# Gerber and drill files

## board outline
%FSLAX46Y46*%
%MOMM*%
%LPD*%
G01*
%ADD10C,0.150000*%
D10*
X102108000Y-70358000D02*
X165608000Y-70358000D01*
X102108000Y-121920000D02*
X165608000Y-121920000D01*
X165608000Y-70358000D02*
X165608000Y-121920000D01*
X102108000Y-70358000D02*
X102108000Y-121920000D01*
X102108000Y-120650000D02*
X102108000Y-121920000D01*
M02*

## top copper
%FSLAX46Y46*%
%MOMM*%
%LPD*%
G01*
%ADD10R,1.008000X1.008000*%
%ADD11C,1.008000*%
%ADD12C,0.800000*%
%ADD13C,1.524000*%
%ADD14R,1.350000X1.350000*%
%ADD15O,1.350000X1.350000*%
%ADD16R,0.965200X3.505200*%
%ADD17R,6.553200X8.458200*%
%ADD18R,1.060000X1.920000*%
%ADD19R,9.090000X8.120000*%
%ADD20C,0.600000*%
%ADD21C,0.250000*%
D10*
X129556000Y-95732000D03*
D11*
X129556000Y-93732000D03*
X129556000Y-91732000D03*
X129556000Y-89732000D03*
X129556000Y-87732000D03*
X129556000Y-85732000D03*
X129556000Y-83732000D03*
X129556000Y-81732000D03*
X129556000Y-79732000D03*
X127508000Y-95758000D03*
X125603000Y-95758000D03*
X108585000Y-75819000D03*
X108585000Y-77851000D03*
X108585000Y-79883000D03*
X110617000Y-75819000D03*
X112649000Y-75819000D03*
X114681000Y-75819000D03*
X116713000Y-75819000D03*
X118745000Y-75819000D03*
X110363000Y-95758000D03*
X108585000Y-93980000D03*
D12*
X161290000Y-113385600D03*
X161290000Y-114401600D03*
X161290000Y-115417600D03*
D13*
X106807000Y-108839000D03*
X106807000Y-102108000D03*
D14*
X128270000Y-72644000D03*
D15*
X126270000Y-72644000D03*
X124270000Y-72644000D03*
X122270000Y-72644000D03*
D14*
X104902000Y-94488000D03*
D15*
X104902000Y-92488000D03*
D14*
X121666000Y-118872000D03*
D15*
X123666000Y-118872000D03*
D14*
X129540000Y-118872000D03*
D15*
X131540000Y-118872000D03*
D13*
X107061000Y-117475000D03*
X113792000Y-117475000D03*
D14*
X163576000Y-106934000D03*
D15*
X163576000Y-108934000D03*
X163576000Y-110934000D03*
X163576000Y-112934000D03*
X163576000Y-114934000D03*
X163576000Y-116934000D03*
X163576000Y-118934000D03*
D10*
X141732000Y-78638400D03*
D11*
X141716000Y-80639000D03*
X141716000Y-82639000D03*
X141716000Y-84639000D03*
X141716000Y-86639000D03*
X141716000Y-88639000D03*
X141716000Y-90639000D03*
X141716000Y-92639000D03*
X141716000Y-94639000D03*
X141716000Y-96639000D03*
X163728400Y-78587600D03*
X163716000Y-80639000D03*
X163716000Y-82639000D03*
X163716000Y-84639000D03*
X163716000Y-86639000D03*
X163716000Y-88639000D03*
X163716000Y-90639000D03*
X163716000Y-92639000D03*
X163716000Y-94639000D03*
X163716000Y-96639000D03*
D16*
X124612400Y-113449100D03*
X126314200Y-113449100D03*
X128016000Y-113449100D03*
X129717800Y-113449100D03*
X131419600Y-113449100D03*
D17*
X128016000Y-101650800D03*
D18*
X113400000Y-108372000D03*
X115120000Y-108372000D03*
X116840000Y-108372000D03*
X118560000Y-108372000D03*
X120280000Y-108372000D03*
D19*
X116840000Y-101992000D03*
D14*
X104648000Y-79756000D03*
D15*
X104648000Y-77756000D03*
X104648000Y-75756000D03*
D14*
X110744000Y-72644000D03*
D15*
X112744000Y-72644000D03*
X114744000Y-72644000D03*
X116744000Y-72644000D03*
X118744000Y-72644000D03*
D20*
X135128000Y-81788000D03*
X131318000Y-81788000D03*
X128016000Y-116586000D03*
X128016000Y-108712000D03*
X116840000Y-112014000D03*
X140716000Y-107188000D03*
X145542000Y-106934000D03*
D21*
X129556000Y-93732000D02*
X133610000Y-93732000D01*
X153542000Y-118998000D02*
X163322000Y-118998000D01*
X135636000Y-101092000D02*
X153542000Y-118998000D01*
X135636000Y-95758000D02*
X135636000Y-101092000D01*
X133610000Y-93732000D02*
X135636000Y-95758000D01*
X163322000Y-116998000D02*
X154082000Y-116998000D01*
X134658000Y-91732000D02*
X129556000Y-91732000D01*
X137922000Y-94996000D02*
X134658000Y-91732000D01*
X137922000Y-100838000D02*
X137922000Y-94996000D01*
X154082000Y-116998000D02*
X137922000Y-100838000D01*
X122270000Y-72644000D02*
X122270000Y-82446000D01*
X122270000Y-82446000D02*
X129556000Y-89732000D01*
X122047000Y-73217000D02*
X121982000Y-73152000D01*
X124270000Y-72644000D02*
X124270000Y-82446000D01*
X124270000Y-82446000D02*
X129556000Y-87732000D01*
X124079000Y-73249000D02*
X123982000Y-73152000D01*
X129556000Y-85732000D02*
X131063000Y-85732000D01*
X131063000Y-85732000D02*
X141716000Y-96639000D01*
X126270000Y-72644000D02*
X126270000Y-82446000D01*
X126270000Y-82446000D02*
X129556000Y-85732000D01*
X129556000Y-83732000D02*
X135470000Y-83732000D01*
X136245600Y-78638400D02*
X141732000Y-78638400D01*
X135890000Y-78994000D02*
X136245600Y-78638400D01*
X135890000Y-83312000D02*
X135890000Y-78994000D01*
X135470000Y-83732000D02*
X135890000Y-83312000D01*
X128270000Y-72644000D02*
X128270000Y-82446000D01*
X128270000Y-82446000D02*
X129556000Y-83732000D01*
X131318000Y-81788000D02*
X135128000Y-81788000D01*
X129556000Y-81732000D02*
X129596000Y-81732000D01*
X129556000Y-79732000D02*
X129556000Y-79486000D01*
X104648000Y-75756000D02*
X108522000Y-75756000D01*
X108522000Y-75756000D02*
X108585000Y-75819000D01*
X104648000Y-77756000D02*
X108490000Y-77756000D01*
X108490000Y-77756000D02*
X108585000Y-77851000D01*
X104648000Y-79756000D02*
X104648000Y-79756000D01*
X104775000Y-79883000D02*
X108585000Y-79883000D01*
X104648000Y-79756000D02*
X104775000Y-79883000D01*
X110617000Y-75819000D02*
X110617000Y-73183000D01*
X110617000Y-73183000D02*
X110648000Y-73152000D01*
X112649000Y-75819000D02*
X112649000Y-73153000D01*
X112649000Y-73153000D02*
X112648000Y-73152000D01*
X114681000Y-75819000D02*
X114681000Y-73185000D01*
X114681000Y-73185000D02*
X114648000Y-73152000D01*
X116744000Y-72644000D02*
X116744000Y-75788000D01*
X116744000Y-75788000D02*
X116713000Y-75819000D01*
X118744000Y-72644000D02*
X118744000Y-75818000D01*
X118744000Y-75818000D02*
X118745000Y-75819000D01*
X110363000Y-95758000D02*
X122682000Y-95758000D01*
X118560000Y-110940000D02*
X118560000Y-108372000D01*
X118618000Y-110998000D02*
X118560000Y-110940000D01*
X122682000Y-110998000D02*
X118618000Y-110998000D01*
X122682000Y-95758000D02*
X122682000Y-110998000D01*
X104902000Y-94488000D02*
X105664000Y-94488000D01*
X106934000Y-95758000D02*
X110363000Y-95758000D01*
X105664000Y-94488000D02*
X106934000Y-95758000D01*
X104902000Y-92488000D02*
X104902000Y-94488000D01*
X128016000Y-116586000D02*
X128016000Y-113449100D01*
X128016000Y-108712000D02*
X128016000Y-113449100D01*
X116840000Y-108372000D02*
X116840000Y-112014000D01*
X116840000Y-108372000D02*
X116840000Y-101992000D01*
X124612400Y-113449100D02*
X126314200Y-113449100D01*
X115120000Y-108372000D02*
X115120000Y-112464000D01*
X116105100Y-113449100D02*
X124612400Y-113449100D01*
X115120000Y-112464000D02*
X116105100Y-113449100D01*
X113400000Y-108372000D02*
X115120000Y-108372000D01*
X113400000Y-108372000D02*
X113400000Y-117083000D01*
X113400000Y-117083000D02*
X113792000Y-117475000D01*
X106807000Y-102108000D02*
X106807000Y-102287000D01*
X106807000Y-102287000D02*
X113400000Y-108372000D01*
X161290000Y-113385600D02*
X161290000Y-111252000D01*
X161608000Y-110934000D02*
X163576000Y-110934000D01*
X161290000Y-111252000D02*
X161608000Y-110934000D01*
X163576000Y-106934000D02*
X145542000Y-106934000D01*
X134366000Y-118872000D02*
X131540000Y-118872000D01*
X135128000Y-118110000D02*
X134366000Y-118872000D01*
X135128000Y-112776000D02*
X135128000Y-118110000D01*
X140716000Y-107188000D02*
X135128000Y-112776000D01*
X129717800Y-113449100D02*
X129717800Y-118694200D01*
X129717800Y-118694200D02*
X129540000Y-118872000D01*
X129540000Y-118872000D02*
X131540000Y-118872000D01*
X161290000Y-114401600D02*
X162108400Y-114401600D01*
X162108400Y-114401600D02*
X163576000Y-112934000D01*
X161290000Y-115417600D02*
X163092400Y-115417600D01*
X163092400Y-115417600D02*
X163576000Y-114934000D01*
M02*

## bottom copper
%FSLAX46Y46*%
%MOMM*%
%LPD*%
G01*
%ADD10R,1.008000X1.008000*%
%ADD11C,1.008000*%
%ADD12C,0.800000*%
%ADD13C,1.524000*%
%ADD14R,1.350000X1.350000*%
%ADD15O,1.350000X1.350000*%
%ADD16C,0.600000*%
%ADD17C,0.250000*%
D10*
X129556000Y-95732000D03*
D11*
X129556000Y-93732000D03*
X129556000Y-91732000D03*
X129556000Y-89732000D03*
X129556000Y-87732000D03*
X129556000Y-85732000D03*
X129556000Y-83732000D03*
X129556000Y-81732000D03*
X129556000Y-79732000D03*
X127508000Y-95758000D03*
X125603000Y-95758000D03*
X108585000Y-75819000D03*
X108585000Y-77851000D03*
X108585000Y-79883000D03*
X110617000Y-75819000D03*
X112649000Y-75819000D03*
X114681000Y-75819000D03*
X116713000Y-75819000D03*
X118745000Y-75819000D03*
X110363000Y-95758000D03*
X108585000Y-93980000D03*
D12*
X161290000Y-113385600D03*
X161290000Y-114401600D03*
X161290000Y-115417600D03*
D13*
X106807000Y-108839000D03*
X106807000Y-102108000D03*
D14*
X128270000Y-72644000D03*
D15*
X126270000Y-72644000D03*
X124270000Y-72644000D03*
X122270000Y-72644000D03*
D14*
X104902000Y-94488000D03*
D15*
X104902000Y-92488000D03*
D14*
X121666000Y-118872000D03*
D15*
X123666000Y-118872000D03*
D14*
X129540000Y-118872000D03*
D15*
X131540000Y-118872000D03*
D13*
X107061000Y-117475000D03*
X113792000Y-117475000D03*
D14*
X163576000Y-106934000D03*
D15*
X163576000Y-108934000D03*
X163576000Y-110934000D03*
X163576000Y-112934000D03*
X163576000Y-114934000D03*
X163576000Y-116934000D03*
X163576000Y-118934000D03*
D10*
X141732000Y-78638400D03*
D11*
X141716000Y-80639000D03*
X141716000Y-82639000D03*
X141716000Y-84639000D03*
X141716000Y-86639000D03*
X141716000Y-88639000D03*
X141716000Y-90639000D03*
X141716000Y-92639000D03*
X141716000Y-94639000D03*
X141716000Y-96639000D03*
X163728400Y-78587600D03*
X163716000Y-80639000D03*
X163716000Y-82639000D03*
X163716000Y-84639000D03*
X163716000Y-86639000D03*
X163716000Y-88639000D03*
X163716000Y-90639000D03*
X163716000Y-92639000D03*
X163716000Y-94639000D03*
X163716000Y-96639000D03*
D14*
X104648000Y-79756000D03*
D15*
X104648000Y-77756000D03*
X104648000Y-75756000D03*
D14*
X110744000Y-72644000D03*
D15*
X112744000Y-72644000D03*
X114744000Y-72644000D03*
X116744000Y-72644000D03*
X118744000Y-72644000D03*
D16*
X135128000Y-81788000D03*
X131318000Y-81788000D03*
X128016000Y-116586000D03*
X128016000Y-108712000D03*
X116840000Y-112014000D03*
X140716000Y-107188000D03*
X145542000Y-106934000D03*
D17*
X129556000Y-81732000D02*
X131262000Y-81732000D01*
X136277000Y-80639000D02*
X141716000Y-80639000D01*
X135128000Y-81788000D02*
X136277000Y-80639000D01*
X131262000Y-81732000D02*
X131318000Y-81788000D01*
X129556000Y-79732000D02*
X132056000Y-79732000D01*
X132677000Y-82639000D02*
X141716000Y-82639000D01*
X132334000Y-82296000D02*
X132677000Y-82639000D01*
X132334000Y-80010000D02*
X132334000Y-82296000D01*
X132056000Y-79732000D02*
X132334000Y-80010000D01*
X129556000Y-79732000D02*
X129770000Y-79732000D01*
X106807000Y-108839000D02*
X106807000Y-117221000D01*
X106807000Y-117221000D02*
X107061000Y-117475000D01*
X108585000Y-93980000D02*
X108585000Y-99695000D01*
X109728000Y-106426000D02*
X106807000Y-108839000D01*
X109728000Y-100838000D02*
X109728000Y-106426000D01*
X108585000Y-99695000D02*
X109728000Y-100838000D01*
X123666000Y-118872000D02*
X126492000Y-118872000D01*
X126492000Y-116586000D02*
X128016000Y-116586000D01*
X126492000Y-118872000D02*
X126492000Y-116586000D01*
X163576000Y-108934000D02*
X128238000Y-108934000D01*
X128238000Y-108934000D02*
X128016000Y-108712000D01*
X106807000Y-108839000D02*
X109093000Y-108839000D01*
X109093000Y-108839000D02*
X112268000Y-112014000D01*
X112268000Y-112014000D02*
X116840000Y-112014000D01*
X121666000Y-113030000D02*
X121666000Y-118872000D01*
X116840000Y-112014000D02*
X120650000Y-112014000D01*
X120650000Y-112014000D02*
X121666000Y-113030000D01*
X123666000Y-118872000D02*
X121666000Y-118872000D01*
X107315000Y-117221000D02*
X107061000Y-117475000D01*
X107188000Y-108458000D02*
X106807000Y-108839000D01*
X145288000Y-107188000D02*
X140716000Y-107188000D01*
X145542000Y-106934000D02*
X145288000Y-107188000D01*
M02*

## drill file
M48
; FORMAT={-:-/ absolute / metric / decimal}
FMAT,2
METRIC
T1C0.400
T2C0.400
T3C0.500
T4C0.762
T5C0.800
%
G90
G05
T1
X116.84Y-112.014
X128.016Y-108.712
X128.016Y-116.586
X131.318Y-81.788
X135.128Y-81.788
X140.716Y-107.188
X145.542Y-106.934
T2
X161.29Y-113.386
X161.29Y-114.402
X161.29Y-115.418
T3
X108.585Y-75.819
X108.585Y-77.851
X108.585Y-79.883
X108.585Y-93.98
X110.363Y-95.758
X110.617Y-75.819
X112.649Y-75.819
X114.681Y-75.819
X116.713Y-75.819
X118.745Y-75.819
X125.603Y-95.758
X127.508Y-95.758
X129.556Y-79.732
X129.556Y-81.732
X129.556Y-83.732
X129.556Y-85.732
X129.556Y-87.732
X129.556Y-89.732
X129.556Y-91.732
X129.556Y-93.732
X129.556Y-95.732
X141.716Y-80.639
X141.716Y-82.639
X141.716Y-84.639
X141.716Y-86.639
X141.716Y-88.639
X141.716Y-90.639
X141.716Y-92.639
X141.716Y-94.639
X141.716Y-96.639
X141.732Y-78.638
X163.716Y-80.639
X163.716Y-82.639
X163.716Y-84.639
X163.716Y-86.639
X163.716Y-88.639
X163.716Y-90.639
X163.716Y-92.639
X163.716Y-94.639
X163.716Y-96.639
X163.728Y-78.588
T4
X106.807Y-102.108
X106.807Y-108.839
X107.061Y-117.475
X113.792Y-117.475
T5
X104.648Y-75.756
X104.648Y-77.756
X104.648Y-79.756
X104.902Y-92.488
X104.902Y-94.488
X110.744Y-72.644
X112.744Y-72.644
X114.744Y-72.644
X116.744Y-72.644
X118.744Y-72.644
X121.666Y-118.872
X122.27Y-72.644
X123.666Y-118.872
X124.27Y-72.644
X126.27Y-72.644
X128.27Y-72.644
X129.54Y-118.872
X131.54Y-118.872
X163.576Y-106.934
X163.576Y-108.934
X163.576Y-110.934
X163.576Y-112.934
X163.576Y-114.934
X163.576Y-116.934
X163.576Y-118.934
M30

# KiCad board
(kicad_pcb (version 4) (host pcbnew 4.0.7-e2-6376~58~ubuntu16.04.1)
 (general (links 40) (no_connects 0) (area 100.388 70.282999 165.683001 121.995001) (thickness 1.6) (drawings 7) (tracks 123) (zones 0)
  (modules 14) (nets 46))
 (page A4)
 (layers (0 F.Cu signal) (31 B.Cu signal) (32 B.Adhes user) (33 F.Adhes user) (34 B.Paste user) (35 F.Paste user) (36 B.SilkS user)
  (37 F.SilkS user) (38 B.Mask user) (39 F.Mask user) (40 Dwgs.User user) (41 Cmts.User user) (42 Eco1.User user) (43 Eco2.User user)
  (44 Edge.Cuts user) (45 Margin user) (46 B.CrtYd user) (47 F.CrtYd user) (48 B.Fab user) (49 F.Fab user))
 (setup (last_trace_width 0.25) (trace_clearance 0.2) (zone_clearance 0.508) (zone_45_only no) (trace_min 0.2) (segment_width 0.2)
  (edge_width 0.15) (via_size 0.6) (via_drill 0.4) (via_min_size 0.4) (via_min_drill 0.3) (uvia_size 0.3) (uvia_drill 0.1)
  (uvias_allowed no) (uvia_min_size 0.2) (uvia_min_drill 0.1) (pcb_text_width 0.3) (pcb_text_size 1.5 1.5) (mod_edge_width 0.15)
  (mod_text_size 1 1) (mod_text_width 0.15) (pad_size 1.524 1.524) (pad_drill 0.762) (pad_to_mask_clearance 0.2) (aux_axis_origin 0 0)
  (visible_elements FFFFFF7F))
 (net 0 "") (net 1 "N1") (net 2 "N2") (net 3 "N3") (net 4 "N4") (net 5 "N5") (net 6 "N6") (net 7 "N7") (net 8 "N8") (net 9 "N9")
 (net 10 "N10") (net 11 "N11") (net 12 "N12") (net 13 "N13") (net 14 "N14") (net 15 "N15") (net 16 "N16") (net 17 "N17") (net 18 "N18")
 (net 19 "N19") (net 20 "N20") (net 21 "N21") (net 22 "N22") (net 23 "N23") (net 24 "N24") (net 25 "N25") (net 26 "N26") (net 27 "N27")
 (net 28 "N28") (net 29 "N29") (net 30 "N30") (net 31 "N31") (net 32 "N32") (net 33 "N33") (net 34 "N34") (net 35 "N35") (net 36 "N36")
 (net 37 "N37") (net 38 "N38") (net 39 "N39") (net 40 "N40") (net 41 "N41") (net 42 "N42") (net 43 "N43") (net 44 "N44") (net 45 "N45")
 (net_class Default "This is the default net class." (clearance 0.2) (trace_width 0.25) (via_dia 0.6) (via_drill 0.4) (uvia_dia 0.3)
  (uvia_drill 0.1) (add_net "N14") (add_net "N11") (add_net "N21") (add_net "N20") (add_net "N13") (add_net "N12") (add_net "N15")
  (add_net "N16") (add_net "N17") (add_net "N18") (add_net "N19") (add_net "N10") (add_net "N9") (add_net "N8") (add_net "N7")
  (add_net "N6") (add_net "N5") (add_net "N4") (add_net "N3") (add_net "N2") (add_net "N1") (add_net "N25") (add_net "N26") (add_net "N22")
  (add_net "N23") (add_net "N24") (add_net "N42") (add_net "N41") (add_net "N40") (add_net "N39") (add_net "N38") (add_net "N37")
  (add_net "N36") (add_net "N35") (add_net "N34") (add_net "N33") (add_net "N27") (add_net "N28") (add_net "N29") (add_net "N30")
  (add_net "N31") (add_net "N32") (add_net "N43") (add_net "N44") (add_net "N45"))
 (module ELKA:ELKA (layer F.Cu) (at 118.11 72.39 180)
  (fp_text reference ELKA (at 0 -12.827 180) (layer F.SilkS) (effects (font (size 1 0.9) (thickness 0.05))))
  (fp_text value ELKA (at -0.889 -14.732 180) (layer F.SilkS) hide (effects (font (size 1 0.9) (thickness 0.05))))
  (pad I thru_hole rect (at -11.446 -23.342 180) (size 1.008 1.008) (drill 0.5) (layers *.Cu *.Mask F.SilkS) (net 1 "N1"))
  (pad H thru_hole circle (at -11.446 -21.342 180) (size 1.008 1.008) (drill 0.5) (layers *.Cu *.Mask F.SilkS) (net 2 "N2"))
  (pad G thru_hole circle (at -11.446 -19.342 180) (size 1.008 1.008) (drill 0.5) (layers *.Cu *.Mask F.SilkS) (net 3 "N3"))
  (pad F thru_hole circle (at -11.446 -17.342 180) (size 1.008 1.008) (drill 0.5) (layers *.Cu *.Mask F.SilkS) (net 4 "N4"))
  (pad E thru_hole circle (at -11.446 -15.342 180) (size 1.008 1.008) (drill 0.5) (layers *.Cu *.Mask F.SilkS) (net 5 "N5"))
  (pad D thru_hole circle (at -11.446 -13.342 180) (size 1.008 1.008) (drill 0.5) (layers *.Cu *.Mask F.SilkS) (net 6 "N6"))
  (pad C thru_hole circle (at -11.446 -11.342 180) (size 1.008 1.008) (drill 0.5) (layers *.Cu *.Mask F.SilkS) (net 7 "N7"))
  (pad B thru_hole circle (at -11.446 -9.342 180) (size 1.008 1.008) (drill 0.5) (layers *.Cu *.Mask F.SilkS) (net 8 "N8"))
  (pad A thru_hole circle (at -11.446 -7.342 180) (size 1.008 1.008) (drill 0.5) (layers *.Cu *.Mask F.SilkS) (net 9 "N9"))
  (pad 9 thru_hole circle (at -9.398 -23.368 180) (size 1.008 1.008) (drill 0.5) (layers *.Cu *.Mask F.SilkS) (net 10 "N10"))
  (pad 10 thru_hole circle (at -7.493 -23.368 180) (size 1.008 1.008) (drill 0.5) (layers *.Cu *.Mask F.SilkS) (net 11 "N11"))
  (pad 3 thru_hole circle (at 9.525 -3.429 180) (size 1.008 1.008) (drill 0.5) (layers *.Cu *.Mask F.SilkS) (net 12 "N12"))
  (pad 2 thru_hole circle (at 9.525 -5.461 180) (size 1.008 1.008) (drill 0.5) (layers *.Cu *.Mask F.SilkS) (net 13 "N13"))
  (pad 1 thru_hole circle (at 9.525 -7.493 180) (size 1.008 1.008) (drill 0.5) (layers *.Cu *.Mask F.SilkS) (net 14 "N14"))
  (pad 4 thru_hole circle (at 7.493 -3.429 180) (size 1.008 1.008) (drill 0.5) (layers *.Cu *.Mask F.SilkS) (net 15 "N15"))
  (pad 5 thru_hole circle (at 5.461 -3.429 180) (size 1.008 1.008) (drill 0.5) (layers *.Cu *.Mask F.SilkS) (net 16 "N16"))
  (pad 6 thru_hole circle (at 3.429 -3.429 180) (size 1.008 1.008) (drill 0.5) (layers *.Cu *.Mask F.SilkS) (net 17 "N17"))
  (pad 7 thru_hole circle (at 1.397 -3.429 180) (size 1.008 1.008) (drill 0.5) (layers *.Cu *.Mask F.SilkS) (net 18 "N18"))
  (pad 8 thru_hole circle (at -0.635 -3.429 180) (size 1.008 1.008) (drill 0.5) (layers *.Cu *.Mask F.SilkS) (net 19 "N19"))
  (pad 12 thru_hole circle (at 7.747 -23.368 180) (size 1.008 1.008) (drill 0.5) (layers *.Cu *.Mask F.SilkS) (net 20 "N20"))
  (pad 11 thru_hole circle (at 9.525 -21.59 180) (size 1.008 1.008) (drill 0.5) (layers *.Cu *.Mask F.SilkS) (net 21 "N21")))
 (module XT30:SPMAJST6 (layer F.Cu) (at 164.084 115.316 270)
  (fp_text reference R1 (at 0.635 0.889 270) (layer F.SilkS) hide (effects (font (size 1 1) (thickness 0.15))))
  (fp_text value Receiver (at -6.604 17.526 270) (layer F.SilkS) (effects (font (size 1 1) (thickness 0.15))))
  (pad 1 thru_hole circle (at -1.9304 2.794 270) (size 0.8 0.8) (drill 0.4) (layers *.Cu *.Mask) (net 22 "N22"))
  (pad 2 thru_hole circle (at -0.9144 2.794 270) (size 0.8 0.8) (drill 0.4) (layers *.Cu *.Mask) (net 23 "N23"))
  (pad 3 thru_hole circle (at 0.1016 2.794 270) (size 0.8 0.8) (drill 0.4) (layers *.Cu *.Mask) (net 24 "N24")))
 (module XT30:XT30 (layer F.Cu) (at 100.838 107.442 90)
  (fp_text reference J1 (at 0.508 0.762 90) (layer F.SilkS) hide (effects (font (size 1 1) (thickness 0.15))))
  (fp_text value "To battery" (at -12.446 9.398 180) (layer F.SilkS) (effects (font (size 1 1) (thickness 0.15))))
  (pad 1 thru_hole circle (at -1.397 5.969 90) (size 1.524 1.524) (drill 0.762) (layers *.Cu *.Mask) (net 21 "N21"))
  (pad 2 thru_hole circle (at 5.334 5.969 90) (size 1.524 1.524) (drill 0.762) (layers *.Cu *.Mask) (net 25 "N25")))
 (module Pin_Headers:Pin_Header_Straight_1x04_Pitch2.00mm (layer F.Cu) (at 128.27 72.644 270)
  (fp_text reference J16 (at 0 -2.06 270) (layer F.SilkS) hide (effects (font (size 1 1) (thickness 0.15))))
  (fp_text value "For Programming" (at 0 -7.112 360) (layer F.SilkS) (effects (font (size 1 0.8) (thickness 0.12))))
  (pad 1 thru_hole rect (at 0 0 270) (size 1.35 1.35) (drill 0.8) (layers *.Cu *.Mask) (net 7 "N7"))
  (pad 2 thru_hole oval (at 0 2 270) (size 1.35 1.35) (drill 0.8) (layers *.Cu *.Mask) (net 6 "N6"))
  (pad 3 thru_hole oval (at 0 4 270) (size 1.35 1.35) (drill 0.8) (layers *.Cu *.Mask) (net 5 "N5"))
  (pad 4 thru_hole oval (at 0 6 270) (size 1.35 1.35) (drill 0.8) (layers *.Cu *.Mask) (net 4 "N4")))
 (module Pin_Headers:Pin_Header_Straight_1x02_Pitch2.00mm (layer F.Cu) (at 104.902 94.488 180)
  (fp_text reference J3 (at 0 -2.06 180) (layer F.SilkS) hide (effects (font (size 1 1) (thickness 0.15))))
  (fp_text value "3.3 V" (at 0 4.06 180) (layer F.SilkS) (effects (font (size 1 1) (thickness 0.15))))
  (pad 1 thru_hole rect (at 0 0 180) (size 1.35 1.35) (drill 0.8) (layers *.Cu *.Mask) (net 20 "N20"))
  (pad 2 thru_hole oval (at 0 2 180) (size 1.35 1.35) (drill 0.8) (layers *.Cu *.Mask) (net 20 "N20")))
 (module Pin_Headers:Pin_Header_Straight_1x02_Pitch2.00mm (layer F.Cu) (at 121.666 118.872 90)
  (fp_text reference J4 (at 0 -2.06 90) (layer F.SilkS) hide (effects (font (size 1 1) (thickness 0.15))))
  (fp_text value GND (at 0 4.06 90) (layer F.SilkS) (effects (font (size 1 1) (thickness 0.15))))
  (pad 1 thru_hole rect (at 0 0 90) (size 1.35 1.35) (drill 0.8) (layers *.Cu *.Mask) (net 21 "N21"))
  (pad 2 thru_hole oval (at 0 2 90) (size 1.35 1.35) (drill 0.8) (layers *.Cu *.Mask) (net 21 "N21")))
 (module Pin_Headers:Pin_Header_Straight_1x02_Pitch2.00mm (layer F.Cu) (at 129.54 118.872 90)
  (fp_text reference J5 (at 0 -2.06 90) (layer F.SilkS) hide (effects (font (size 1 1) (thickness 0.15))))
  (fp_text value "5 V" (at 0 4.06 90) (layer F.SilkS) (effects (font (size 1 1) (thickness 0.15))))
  (pad 1 thru_hole rect (at 0 0 90) (size 1.35 1.35) (drill 0.8) (layers *.Cu *.Mask) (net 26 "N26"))
  (pad 2 thru_hole oval (at 0 2 90) (size 1.35 1.35) (drill 0.8) (layers *.Cu *.Mask) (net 26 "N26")))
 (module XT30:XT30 (layer F.Cu) (at 108.458 111.506)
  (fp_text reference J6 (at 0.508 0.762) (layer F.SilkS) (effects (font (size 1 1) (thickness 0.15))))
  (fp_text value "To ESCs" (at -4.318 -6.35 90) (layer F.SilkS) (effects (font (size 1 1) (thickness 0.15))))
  (pad 1 thru_hole circle (at -1.397 5.969) (size 1.524 1.524) (drill 0.762) (layers *.Cu *.Mask) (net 21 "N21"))
  (pad 2 thru_hole circle (at 5.334 5.969) (size 1.524 1.524) (drill 0.762) (layers *.Cu *.Mask) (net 25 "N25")))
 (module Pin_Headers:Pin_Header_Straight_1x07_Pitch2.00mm (layer F.Cu) (at 163.576 106.934)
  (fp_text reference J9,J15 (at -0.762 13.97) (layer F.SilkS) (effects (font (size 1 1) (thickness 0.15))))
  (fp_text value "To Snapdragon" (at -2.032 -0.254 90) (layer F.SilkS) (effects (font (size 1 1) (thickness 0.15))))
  (pad 1 thru_hole rect (at 0 0) (size 1.35 1.35) (drill 0.8) (layers *.Cu *.Mask) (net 26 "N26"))
  (pad 2 thru_hole oval (at 0 2) (size 1.35 1.35) (drill 0.8) (layers *.Cu *.Mask) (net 21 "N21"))
  (pad 3 thru_hole oval (at 0 4) (size 1.35 1.35) (drill 0.8) (layers *.Cu *.Mask) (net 22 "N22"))
  (pad 4 thru_hole oval (at 0 6) (size 1.35 1.35) (drill 0.8) (layers *.Cu *.Mask) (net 23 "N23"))
  (pad 5 thru_hole oval (at 0 8) (size 1.35 1.35) (drill 0.8) (layers *.Cu *.Mask) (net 24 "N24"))
  (pad 6 thru_hole oval (at 0 10) (size 1.35 1.35) (drill 0.8) (layers *.Cu *.Mask) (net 3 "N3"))
  (pad 7 thru_hole oval (at 0 12) (size 1.35 1.35) (drill 0.8) (layers *.Cu *.Mask) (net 2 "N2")))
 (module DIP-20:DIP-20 (layer F.Cu) (at 140.462 104.648)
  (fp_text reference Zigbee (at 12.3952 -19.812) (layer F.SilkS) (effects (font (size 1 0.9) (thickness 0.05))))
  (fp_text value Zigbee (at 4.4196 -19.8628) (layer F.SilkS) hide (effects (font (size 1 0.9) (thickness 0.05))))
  (pad 1 thru_hole rect (at 1.27 -26.0096) (size 1.008 1.008) (drill 0.5) (layers *.Cu *.Mask F.SilkS) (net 7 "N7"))
  (pad 2 thru_hole circle (at 1.254 -24.009) (size 1.008 1.008) (drill 0.5) (layers *.Cu *.Mask F.SilkS) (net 8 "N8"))
  (pad 3 thru_hole circle (at 1.254 -22.009) (size 1.008 1.008) (drill 0.5) (layers *.Cu *.Mask F.SilkS) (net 9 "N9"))
  (pad 4 thru_hole circle (at 1.254 -20.009) (size 1.008 1.008) (drill 0.5) (layers *.Cu *.Mask F.SilkS) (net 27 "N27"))
  (pad 5 thru_hole circle (at 1.254 -18.009) (size 1.008 1.008) (drill 0.5) (layers *.Cu *.Mask F.SilkS) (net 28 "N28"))
  (pad 6 thru_hole circle (at 1.254 -16.009) (size 1.008 1.008) (drill 0.5) (layers *.Cu *.Mask F.SilkS) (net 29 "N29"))
  (pad 7 thru_hole circle (at 1.254 -14.009) (size 1.008 1.008) (drill 0.5) (layers *.Cu *.Mask F.SilkS) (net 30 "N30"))
  (pad 8 thru_hole circle (at 1.254 -12.009) (size 1.008 1.008) (drill 0.5) (layers *.Cu *.Mask F.SilkS) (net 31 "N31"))
  (pad 9 thru_hole circle (at 1.254 -10.009) (size 1.008 1.008) (drill 0.5) (layers *.Cu *.Mask F.SilkS) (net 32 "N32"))
  (pad 10 thru_hole circle (at 1.254 -8.009) (size 1.008 1.008) (drill 0.5) (layers *.Cu *.Mask F.SilkS) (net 6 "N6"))
  (pad 20 thru_hole circle (at 23.2664 -26.0604) (size 1.008 1.008) (drill 0.5) (layers *.Cu *.Mask F.SilkS) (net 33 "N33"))
  (pad 19 thru_hole circle (at 23.254 -24.009) (size 1.008 1.008) (drill 0.5) (layers *.Cu *.Mask F.SilkS) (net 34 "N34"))
  (pad 18 thru_hole circle (at 23.254 -22.009) (size 1.008 1.008) (drill 0.5) (layers *.Cu *.Mask F.SilkS) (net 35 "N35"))
  (pad 17 thru_hole circle (at 23.254 -20.009) (size 1.008 1.008) (drill 0.5) (layers *.Cu *.Mask F.SilkS) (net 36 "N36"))
  (pad 16 thru_hole circle (at 23.254 -18.009) (size 1.008 1.008) (drill 0.5) (layers *.Cu *.Mask F.SilkS) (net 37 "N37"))
  (pad 15 thru_hole circle (at 23.254 -16.009) (size 1.008 1.008) (drill 0.5) (layers *.Cu *.Mask F.SilkS) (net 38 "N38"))
  (pad 14 thru_hole circle (at 23.254 -14.009) (size 1.008 1.008) (drill 0.5) (layers *.Cu *.Mask F.SilkS) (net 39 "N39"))
  (pad 13 thru_hole circle (at 23.254 -12.009) (size 1.008 1.008) (drill 0.5) (layers *.Cu *.Mask F.SilkS) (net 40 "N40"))
  (pad 12 thru_hole circle (at 23.254 -10.009) (size 1.008 1.008) (drill 0.5) (layers *.Cu *.Mask F.SilkS) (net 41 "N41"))
  (pad 11 thru_hole circle (at 23.254 -8.009) (size 1.008 1.008) (drill 0.5) (layers *.Cu *.Mask F.SilkS) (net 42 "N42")))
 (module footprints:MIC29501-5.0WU (layer F.Cu) (at 128.016 104.394)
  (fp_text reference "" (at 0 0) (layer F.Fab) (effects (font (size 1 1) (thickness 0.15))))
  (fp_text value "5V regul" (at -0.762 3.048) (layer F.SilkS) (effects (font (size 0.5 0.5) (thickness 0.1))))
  (pad 1 smd rect (at -3.4036 9.0551) (size 0.9652 3.5052) (layers F.Cu F.Paste F.Mask) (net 25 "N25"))
  (pad 2 smd rect (at -1.7018 9.0551) (size 0.9652 3.5052) (layers F.Cu F.Paste F.Mask) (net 25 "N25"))
  (pad 3 smd rect (at 0 9.0551) (size 0.9652 3.5052) (layers F.Cu F.Paste F.Mask) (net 21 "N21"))
  (pad 4 smd rect (at 1.7018 9.0551) (size 0.9652 3.5052) (layers F.Cu F.Paste F.Mask) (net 26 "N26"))
  (pad 5 smd rect (at 3.4036 9.0551) (size 0.9652 3.5052) (layers F.Cu F.Paste F.Mask) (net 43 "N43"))
  (pad 6 smd rect (at 0 -2.7432) (size 6.5532 8.4582) (layers F.Cu F.Paste F.Mask) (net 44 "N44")))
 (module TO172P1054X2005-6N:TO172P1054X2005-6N (layer F.Cu) (at 116.84 103.632)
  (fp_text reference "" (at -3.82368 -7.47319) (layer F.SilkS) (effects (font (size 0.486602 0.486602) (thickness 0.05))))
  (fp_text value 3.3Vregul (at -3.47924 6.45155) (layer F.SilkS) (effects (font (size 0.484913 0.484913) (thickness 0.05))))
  (pad 1 smd rect (at -3.44 4.74 90) (size 1.92 1.06) (layers F.Cu F.Paste F.Mask) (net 25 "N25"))
  (pad 2 smd rect (at -1.72 4.74 90) (size 1.92 1.06) (layers F.Cu F.Paste F.Mask) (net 25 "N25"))
  (pad 3 smd rect (at 0 4.74 90) (size 1.92 1.06) (layers F.Cu F.Paste F.Mask) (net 21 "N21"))
  (pad 4 smd rect (at 1.72 4.74 90) (size 1.92 1.06) (layers F.Cu F.Paste F.Mask) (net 20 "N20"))
  (pad 5 smd rect (at 3.44 4.74 90) (size 1.92 1.06) (layers F.Cu F.Paste F.Mask) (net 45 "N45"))
  (pad 6 smd rect (at 0 -1.64 90) (size 8.12 9.09) (layers F.Cu F.Paste F.Mask) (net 21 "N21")))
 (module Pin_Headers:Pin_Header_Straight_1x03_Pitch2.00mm (layer F.Cu) (at 104.648 79.756 180)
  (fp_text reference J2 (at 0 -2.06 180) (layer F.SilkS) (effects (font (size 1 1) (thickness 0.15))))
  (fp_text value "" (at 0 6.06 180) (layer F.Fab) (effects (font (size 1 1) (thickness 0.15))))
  (pad 1 thru_hole rect (at 0 0 180) (size 1.35 1.35) (drill 0.8) (layers *.Cu *.Mask) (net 14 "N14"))
  (pad 2 thru_hole oval (at 0 2 180) (size 1.35 1.35) (drill 0.8) (layers *.Cu *.Mask) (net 13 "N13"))
  (pad 3 thru_hole oval (at 0 4 180) (size 1.35 1.35) (drill 0.8) (layers *.Cu *.Mask) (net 12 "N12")))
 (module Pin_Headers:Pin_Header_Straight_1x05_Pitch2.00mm (layer F.Cu) (at 110.744 72.644 90)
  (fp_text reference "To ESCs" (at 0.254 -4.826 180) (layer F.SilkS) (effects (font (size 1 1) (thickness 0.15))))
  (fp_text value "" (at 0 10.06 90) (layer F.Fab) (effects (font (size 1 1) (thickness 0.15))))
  (pad 1 thru_hole rect (at 0 0 90) (size 1.35 1.35) (drill 0.8) (layers *.Cu *.Mask) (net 15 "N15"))
  (pad 2 thru_hole oval (at 0 2 90) (size 1.35 1.35) (drill 0.8) (layers *.Cu *.Mask) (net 16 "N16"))
  (pad 3 thru_hole oval (at 0 4 90) (size 1.35 1.35) (drill 0.8) (layers *.Cu *.Mask) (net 17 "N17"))
  (pad 4 thru_hole oval (at 0 6 90) (size 1.35 1.35) (drill 0.8) (layers *.Cu *.Mask) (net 18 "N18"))
  (pad 5 thru_hole oval (at 0 8 90) (size 1.35 1.35) (drill 0.8) (layers *.Cu *.Mask) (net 19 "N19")))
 (gr_line (start 102.108 70.358) (end 165.608 70.358) (angle 90) (layer Edge.Cuts) (width 0.15))
 (gr_line (start 102.108 121.92) (end 165.608 121.92) (angle 90) (layer Edge.Cuts) (width 0.15))
 (gr_line (start 165.608 70.358) (end 165.608 121.92) (angle 90) (layer Edge.Cuts) (width 0.15))
 (gr_line (start 102.108 70.358) (end 102.108 121.92) (angle 90) (layer Edge.Cuts) (width 0.15))
 (gr_line (start 102.108 120.65) (end 102.108 121.92) (angle 90) (layer Edge.Cuts) (width 0.15))
 (segment (start 129.556 93.732) (end 133.61 93.732) (width 0.25) (layer F.Cu) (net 2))
 (segment (start 153.542 118.998) (end 163.322 118.998) (width 0.25) (layer F.Cu) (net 2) (status 20))
 (segment (start 135.636 101.092) (end 153.542 118.998) (width 0.25) (layer F.Cu) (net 2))
 (segment (start 135.636 95.758) (end 135.636 101.092) (width 0.25) (layer F.Cu) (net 2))
 (segment (start 133.61 93.732) (end 135.636 95.758) (width 0.25) (layer F.Cu) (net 2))
 (segment (start 163.322 116.998) (end 154.082 116.998) (width 0.25) (layer F.Cu) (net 3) (status 10))
 (segment (start 134.658 91.732) (end 129.556 91.732) (width 0.25) (layer F.Cu) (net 3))
 (segment (start 137.922 94.996) (end 134.658 91.732) (width 0.25) (layer F.Cu) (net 3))
 (segment (start 137.922 100.838) (end 137.922 94.996) (width 0.25) (layer F.Cu) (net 3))
 (segment (start 154.082 116.998) (end 137.922 100.838) (width 0.25) (layer F.Cu) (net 3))
 (segment (start 122.27 72.644) (end 122.27 82.446) (width 0.25) (layer F.Cu) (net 4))
 (segment (start 122.27 82.446) (end 129.556 89.732) (width 0.25) (layer F.Cu) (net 4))
 (segment (start 122.047 73.217) (end 121.982 73.152) (width 0.25) (layer F.Cu) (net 4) (status 30))
 (segment (start 124.27 72.644) (end 124.27 82.446) (width 0.25) (layer F.Cu) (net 5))
 (segment (start 124.27 82.446) (end 129.556 87.732) (width 0.25) (layer F.Cu) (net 5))
 (segment (start 124.079 73.249) (end 123.982 73.152) (width 0.25) (layer F.Cu) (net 5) (status 30))
 (segment (start 129.556 85.732) (end 131.063 85.732) (width 0.25) (layer F.Cu) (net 6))
 (segment (start 131.063 85.732) (end 141.716 96.639) (width 0.25) (layer F.Cu) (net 6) (status 20))
 (segment (start 126.27 72.644) (end 126.27 82.446) (width 0.25) (layer F.Cu) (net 6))
 (segment (start 126.27 82.446) (end 129.556 85.732) (width 0.25) (layer F.Cu) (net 6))
 (segment (start 129.556 83.732) (end 135.47 83.732) (width 0.25) (layer F.Cu) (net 7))
 (segment (start 136.2456 78.6384) (end 141.732 78.6384) (width 0.25) (layer F.Cu) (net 7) (status 20))
 (segment (start 135.89 78.994) (end 136.2456 78.6384) (width 0.25) (layer F.Cu) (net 7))
 (segment (start 135.89 83.312) (end 135.89 78.994) (width 0.25) (layer F.Cu) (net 7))
 (segment (start 135.47 83.732) (end 135.89 83.312) (width 0.25) (layer F.Cu) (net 7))
 (segment (start 128.27 72.644) (end 128.27 82.446) (width 0.25) (layer F.Cu) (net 7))
 (segment (start 128.27 82.446) (end 129.556 83.732) (width 0.25) (layer F.Cu) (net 7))
 (segment (start 129.556 81.732) (end 131.262 81.732) (width 0.25) (layer B.Cu) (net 8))
 (segment (start 136.277 80.639) (end 141.716 80.639) (width 0.25) (layer B.Cu) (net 8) (status 20))
 (segment (start 135.128 81.788) (end 136.277 80.639) (width 0.25) (layer B.Cu) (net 8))
 (via (at 135.128 81.788) (size 0.6) (drill 0.4) (layers F.Cu B.Cu) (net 8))
 (segment (start 131.318 81.788) (end 135.128 81.788) (width 0.25) (layer F.Cu) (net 8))
 (via (at 131.318 81.788) (size 0.6) (drill 0.4) (layers F.Cu B.Cu) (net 8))
 (segment (start 131.262 81.732) (end 131.318 81.788) (width 0.25) (layer B.Cu) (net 8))
 (segment (start 129.556 81.732) (end 129.596 81.732) (width 0.25) (layer F.Cu) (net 8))
 (segment (start 129.556 79.732) (end 132.056 79.732) (width 0.25) (layer B.Cu) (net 9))
 (segment (start 132.677 82.639) (end 141.716 82.639) (width 0.25) (layer B.Cu) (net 9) (status 20))
 (segment (start 132.334 82.296) (end 132.677 82.639) (width 0.25) (layer B.Cu) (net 9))
 (segment (start 132.334 80.01) (end 132.334 82.296) (width 0.25) (layer B.Cu) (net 9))
 (segment (start 132.056 79.732) (end 132.334 80.01) (width 0.25) (layer B.Cu) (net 9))
 (segment (start 129.556 79.732) (end 129.556 79.486) (width 0.25) (layer F.Cu) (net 9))
 (segment (start 129.556 79.732) (end 129.77 79.732) (width 0.25) (layer B.Cu) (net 9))
 (segment (start 104.648 75.756) (end 108.522 75.756) (width 0.25) (layer F.Cu) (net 12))
 (segment (start 108.522 75.756) (end 108.585 75.819) (width 0.25) (layer F.Cu) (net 12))
 (segment (start 104.648 77.756) (end 108.49 77.756) (width 0.25) (layer F.Cu) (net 13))
 (segment (start 108.49 77.756) (end 108.585 77.851) (width 0.25) (layer F.Cu) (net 13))
 (segment (start 104.648 79.756) (end 104.648 79.756) (width 0.25) (layer F.Cu) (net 14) (status 10))
 (segment (start 104.775 79.883) (end 108.585 79.883) (width 0.25) (layer F.Cu) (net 14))
 (segment (start 104.648 79.756) (end 104.775 79.883) (width 0.25) (layer F.Cu) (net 14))
 (segment (start 110.617 75.819) (end 110.617 73.183) (width 0.25) (layer F.Cu) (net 15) (status 20))
 (segment (start 110.617 73.183) (end 110.648 73.152) (width 0.25) (layer F.Cu) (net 15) (status 30))
 (segment (start 112.649 75.819) (end 112.649 73.153) (width 0.25) (layer F.Cu) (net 16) (status 20))
 (segment (start 112.649 73.153) (end 112.648 73.152) (width 0.25) (layer F.Cu) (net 16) (status 30))
 (segment (start 114.681 75.819) (end 114.681 73.185) (width 0.25) (layer F.Cu) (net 17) (status 20))
 (segment (start 114.681 73.185) (end 114.648 73.152) (width 0.25) (layer F.Cu) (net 17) (status 30))
 (segment (start 116.744 72.644) (end 116.744 75.788) (width 0.25) (layer F.Cu) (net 18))
 (segment (start 116.744 75.788) (end 116.713 75.819) (width 0.25) (layer F.Cu) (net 18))
 (segment (start 118.744 72.644) (end 118.744 75.818) (width 0.25) (layer F.Cu) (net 19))
 (segment (start 118.744 75.818) (end 118.745 75.819) (width 0.25) (layer F.Cu) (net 19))
 (segment (start 110.363 95.758) (end 122.682 95.758) (width 0.25) (layer F.Cu) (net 20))
 (segment (start 118.56 110.94) (end 118.56 108.372) (width 0.25) (layer F.Cu) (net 20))
 (segment (start 118.618 110.998) (end 118.56 110.94) (width 0.25) (layer F.Cu) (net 20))
 (segment (start 122.682 110.998) (end 118.618 110.998) (width 0.25) (layer F.Cu) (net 20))
 (segment (start 122.682 95.758) (end 122.682 110.998) (width 0.25) (layer F.Cu) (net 20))
 (segment (start 104.902 94.488) (end 105.664 94.488) (width 0.25) (layer F.Cu) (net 20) (status 10))
 (segment (start 106.934 95.758) (end 110.363 95.758) (width 0.25) (layer F.Cu) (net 20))
 (segment (start 105.664 94.488) (end 106.934 95.758) (width 0.25) (layer F.Cu) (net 20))
 (segment (start 104.902 92.488) (end 104.902 94.488) (width 0.25) (layer F.Cu) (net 20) (status 30))
 (segment (start 106.807 108.839) (end 106.807 117.221) (width 0.25) (layer B.Cu) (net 21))
 (segment (start 106.807 117.221) (end 107.061 117.475) (width 0.25) (layer B.Cu) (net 21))
 (segment (start 108.585 93.98) (end 108.585 99.695) (width 0.25) (layer B.Cu) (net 21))
 (segment (start 109.728 106.426) (end 106.807 108.839) (width 0.25) (layer B.Cu) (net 21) (status 20))
 (segment (start 109.728 100.838) (end 109.728 106.426) (width 0.25) (layer B.Cu) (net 21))
 (segment (start 108.585 99.695) (end 109.728 100.838) (width 0.25) (layer B.Cu) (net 21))
 (segment (start 123.666 118.872) (end 126.492 118.872) (width 0.25) (layer B.Cu) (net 21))
 (segment (start 128.016 116.586) (end 128.016 113.4491) (width 0.25) (layer F.Cu) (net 21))
 (via (at 128.016 116.586) (size 0.6) (drill 0.4) (layers F.Cu B.Cu) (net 21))
 (segment (start 126.492 116.586) (end 128.016 116.586) (width 0.25) (layer B.Cu) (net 21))
 (segment (start 126.492 118.872) (end 126.492 116.586) (width 0.25) (layer B.Cu) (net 21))
 (segment (start 163.576 108.934) (end 128.238 108.934) (width 0.25) (layer B.Cu) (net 21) (status 10))
 (segment (start 128.238 108.934) (end 128.016 108.712) (width 0.25) (layer B.Cu) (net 21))
 (via (at 128.016 108.712) (size 0.6) (drill 0.4) (layers F.Cu B.Cu) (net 21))
 (segment (start 128.016 108.712) (end 128.016 113.4491) (width 0.25) (layer F.Cu) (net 21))
 (segment (start 116.84 108.372) (end 116.84 112.014) (width 0.25) (layer F.Cu) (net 21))
 (via (at 116.84 112.014) (size 0.6) (drill 0.4) (layers F.Cu B.Cu) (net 21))
 (segment (start 106.807 108.839) (end 109.093 108.839) (width 0.25) (layer B.Cu) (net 21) (status 10))
 (segment (start 109.093 108.839) (end 112.268 112.014) (width 0.25) (layer B.Cu) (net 21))
 (segment (start 112.268 112.014) (end 116.84 112.014) (width 0.25) (layer B.Cu) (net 21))
 (segment (start 121.666 113.03) (end 121.666 118.872) (width 0.25) (layer B.Cu) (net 21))
 (segment (start 116.84 112.014) (end 120.65 112.014) (width 0.25) (layer B.Cu) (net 21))
 (segment (start 120.65 112.014) (end 121.666 113.03) (width 0.25) (layer B.Cu) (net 21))
 (segment (start 123.666 118.872) (end 121.666 118.872) (width 0.25) (layer B.Cu) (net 21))
 (segment (start 107.315 117.221) (end 107.061 117.475) (width 0.25) (layer B.Cu) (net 21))
 (segment (start 107.188 108.458) (end 106.807 108.839) (width 0.25) (layer B.Cu) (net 21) (status 30))
 (segment (start 116.84 108.372) (end 116.84 101.992) (width 0.25) (layer F.Cu) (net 21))
 (segment (start 124.6124 113.4491) (end 126.3142 113.4491) (width 0.25) (layer F.Cu) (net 25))
 (segment (start 115.12 108.372) (end 115.12 112.464) (width 0.25) (layer F.Cu) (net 25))
 (segment (start 116.1051 113.4491) (end 124.6124 113.4491) (width 0.25) (layer F.Cu) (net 25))
 (segment (start 115.12 112.464) (end 116.1051 113.4491) (width 0.25) (layer F.Cu) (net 25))
 (segment (start 113.4 108.372) (end 115.12 108.372) (width 0.25) (layer F.Cu) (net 25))
 (segment (start 113.4 108.372) (end 113.4 117.083) (width 0.25) (layer F.Cu) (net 25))
 (segment (start 113.4 117.083) (end 113.792 117.475) (width 0.25) (layer F.Cu) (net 25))
 (segment (start 106.807 102.108) (end 106.807 102.287) (width 0.25) (layer F.Cu) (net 25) (status 30))
 (segment (start 106.807 102.287) (end 113.4 108.372) (width 0.25) (layer F.Cu) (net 25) (status 10))
 (segment (start 161.29 113.3856) (end 161.29 111.252) (width 0.25) (layer F.Cu) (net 22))
 (segment (start 161.608 110.934) (end 163.576 110.934) (width 0.25) (layer F.Cu) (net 22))
 (segment (start 161.29 111.252) (end 161.608 110.934) (width 0.25) (layer F.Cu) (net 22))
 (segment (start 163.576 106.934) (end 145.542 106.934) (width 0.25) (layer F.Cu) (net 26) (status 10))
 (segment (start 134.366 118.872) (end 131.54 118.872) (width 0.25) (layer F.Cu) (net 26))
 (segment (start 135.128 118.11) (end 134.366 118.872) (width 0.25) (layer F.Cu) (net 26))
 (segment (start 135.128 112.776) (end 135.128 118.11) (width 0.25) (layer F.Cu) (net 26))
 (segment (start 140.716 107.188) (end 135.128 112.776) (width 0.25) (layer F.Cu) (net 26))
 (via (at 140.716 107.188) (size 0.6) (drill 0.4) (layers F.Cu B.Cu) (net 26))
 (segment (start 145.288 107.188) (end 140.716 107.188) (width 0.25) (layer B.Cu) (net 26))
 (segment (start 145.542 106.934) (end 145.288 107.188) (width 0.25) (layer B.Cu) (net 26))
 (via (at 145.542 106.934) (size 0.6) (drill 0.4) (layers F.Cu B.Cu) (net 26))
 (segment (start 129.7178 113.4491) (end 129.7178 118.6942) (width 0.25) (layer F.Cu) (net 26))
 (segment (start 129.7178 118.6942) (end 129.54 118.872) (width 0.25) (layer F.Cu) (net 26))
 (segment (start 129.54 118.872) (end 131.54 118.872) (width 0.25) (layer F.Cu) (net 26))
 (segment (start 161.29 114.4016) (end 162.1084 114.4016) (width 0.25) (layer F.Cu) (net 23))
 (segment (start 162.1084 114.4016) (end 163.576 112.934) (width 0.25) (layer F.Cu) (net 23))
 (segment (start 161.29 115.4176) (end 163.0924 115.4176) (width 0.25) (layer F.Cu) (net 24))
 (segment (start 163.0924 115.4176) (end 163.576 114.934) (width 0.25) (layer F.Cu) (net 24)))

